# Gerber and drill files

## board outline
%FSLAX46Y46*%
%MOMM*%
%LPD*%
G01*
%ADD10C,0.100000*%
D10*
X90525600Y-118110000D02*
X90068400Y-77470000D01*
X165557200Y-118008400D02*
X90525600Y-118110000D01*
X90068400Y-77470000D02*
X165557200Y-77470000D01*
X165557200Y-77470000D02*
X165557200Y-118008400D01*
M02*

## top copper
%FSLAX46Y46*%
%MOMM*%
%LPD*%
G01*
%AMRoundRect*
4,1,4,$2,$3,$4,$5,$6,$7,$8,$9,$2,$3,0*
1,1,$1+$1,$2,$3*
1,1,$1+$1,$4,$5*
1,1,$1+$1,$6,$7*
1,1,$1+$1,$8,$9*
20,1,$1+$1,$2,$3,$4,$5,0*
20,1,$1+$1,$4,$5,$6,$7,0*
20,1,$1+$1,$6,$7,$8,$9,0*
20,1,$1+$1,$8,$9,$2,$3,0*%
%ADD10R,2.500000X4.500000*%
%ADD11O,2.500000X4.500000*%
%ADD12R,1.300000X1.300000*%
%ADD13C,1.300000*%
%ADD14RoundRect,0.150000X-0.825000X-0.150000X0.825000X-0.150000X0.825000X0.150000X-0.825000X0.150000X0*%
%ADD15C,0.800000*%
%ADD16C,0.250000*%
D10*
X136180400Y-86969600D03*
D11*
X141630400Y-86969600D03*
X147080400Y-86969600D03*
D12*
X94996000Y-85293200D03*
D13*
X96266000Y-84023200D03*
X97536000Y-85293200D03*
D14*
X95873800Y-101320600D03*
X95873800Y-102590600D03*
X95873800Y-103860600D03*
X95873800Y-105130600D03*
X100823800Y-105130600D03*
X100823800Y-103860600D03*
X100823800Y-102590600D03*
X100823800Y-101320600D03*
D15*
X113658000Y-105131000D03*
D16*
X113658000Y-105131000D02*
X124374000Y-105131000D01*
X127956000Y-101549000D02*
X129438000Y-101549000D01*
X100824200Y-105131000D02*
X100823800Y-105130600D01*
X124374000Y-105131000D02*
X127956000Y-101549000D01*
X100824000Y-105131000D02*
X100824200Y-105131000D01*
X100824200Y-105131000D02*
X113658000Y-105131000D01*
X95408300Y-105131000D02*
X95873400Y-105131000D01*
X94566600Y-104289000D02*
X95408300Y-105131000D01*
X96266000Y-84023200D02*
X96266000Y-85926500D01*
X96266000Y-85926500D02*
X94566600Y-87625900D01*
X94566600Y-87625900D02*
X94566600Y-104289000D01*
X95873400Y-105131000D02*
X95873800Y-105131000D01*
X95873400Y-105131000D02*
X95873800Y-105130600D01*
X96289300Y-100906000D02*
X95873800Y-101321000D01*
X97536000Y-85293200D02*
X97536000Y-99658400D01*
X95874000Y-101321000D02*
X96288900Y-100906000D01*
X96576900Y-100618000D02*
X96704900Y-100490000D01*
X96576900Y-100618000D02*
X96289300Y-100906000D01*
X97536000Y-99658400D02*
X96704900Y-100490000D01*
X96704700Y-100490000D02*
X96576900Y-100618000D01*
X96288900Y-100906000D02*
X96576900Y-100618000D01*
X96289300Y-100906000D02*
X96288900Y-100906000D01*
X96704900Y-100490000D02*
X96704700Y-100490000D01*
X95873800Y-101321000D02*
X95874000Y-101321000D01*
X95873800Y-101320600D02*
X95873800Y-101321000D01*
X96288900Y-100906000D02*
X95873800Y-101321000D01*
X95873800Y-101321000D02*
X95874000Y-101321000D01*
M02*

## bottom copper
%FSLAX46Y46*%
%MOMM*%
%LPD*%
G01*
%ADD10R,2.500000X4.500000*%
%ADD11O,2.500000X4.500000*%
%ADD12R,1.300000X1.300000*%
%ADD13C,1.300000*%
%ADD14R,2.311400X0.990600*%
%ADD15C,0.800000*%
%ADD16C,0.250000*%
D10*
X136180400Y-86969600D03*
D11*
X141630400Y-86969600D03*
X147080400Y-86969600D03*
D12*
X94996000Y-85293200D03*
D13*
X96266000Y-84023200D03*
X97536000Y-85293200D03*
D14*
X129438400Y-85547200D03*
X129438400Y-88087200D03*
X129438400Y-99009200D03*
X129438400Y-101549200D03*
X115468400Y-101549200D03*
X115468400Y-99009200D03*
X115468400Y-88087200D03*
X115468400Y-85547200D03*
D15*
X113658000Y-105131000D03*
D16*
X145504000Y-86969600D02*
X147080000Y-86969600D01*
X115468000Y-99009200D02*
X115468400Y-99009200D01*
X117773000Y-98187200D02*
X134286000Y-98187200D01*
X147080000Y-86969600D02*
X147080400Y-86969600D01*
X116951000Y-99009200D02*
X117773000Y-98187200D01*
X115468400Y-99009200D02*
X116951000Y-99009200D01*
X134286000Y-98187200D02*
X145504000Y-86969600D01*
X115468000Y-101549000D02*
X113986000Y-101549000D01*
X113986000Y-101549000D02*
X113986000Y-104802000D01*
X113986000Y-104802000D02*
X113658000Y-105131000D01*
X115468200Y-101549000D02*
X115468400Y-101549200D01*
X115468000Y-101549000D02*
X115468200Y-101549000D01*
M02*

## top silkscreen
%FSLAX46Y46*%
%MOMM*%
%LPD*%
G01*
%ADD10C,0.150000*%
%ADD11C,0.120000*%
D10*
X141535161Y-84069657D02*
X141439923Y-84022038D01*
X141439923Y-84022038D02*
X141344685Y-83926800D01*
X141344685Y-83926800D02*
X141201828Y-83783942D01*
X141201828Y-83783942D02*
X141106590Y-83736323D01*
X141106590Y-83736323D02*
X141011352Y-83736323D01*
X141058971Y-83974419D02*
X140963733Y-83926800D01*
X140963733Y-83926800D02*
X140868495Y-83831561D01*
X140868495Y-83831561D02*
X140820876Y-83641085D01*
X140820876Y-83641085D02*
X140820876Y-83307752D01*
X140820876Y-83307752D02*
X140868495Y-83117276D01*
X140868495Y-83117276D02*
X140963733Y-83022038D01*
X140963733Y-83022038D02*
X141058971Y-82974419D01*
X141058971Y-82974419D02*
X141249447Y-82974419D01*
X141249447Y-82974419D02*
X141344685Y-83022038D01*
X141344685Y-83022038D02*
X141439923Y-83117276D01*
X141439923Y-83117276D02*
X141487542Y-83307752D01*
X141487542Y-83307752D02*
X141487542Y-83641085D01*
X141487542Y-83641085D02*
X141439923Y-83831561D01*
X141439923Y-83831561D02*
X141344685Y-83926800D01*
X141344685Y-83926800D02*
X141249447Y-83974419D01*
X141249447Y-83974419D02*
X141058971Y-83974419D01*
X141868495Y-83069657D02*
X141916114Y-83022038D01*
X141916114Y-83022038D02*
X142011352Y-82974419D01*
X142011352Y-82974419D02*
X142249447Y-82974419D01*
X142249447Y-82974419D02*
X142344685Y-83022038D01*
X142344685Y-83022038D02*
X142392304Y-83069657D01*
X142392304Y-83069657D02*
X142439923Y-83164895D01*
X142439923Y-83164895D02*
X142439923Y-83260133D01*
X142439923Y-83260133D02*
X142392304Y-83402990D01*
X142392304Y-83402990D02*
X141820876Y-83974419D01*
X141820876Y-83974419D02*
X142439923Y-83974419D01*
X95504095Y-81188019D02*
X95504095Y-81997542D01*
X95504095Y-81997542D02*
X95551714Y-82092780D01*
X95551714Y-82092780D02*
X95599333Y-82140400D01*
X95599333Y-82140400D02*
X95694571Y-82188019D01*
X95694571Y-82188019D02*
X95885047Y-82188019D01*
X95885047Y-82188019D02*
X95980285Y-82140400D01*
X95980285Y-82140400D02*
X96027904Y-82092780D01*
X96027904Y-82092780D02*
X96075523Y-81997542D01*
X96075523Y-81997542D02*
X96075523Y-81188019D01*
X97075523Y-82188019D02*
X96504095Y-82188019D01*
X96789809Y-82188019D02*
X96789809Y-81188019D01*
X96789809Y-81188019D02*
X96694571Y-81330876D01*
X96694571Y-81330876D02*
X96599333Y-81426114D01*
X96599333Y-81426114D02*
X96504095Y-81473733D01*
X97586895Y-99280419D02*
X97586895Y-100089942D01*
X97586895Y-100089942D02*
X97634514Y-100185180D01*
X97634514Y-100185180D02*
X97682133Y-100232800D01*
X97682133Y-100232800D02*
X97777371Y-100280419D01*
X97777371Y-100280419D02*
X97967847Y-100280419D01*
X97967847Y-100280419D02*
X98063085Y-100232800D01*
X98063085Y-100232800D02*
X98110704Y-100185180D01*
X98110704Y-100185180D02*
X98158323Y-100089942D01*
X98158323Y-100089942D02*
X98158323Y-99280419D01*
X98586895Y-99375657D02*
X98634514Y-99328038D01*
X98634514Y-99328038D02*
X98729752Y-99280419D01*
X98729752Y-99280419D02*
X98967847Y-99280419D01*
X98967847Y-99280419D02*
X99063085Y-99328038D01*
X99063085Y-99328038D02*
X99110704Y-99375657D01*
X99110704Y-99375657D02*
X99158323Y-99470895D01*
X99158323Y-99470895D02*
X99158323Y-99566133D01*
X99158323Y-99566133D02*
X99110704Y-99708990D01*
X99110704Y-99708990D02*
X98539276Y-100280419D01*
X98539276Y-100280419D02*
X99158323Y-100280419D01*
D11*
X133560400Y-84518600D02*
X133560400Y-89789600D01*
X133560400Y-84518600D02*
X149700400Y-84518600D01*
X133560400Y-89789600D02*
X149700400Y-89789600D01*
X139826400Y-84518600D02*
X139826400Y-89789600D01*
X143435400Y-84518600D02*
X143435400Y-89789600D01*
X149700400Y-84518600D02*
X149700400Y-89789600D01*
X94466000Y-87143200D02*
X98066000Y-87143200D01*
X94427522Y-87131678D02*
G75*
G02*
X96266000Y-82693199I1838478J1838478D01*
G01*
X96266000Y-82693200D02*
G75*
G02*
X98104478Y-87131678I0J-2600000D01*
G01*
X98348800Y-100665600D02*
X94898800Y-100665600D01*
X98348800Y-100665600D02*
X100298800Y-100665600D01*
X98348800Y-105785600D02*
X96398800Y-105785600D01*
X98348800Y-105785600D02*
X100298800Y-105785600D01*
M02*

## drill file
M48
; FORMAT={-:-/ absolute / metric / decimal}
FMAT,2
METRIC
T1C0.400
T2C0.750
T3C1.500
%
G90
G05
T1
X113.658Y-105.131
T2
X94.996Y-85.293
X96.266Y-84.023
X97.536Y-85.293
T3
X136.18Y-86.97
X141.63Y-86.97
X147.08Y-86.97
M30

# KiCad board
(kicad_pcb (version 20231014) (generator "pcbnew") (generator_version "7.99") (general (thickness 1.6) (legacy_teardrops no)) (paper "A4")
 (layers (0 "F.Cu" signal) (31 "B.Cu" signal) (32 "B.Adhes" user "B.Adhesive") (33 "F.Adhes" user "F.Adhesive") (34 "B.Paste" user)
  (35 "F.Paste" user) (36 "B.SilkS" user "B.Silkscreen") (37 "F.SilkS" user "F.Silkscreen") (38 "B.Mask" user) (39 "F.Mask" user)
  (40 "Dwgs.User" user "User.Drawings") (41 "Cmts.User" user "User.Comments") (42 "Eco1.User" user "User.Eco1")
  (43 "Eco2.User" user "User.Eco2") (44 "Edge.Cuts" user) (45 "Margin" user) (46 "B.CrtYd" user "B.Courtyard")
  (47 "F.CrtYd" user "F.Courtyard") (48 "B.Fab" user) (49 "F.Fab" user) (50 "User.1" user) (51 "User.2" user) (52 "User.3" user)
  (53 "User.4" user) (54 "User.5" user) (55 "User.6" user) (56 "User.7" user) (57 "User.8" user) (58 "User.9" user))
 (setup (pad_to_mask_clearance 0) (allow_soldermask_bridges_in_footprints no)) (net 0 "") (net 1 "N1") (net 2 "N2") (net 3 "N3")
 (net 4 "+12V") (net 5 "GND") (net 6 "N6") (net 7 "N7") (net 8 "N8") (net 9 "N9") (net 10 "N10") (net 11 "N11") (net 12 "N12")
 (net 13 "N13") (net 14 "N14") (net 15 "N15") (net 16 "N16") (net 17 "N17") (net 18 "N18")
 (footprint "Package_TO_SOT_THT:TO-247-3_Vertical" (layer "F.Cu") (at 136.1804 86.9696)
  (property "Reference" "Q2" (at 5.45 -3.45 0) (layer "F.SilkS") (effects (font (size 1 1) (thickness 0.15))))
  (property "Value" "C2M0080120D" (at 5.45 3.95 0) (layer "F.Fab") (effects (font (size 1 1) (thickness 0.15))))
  (fp_line (start -2.62 -2.451) (end -2.62 2.82) (stroke (width 0.12) (type solid)) (layer "F.SilkS"))
  (fp_line (start -2.62 -2.451) (end 13.52 -2.451) (stroke (width 0.12) (type solid)) (layer "F.SilkS"))
  (fp_line (start -2.62 2.82) (end 13.52 2.82) (stroke (width 0.12) (type solid)) (layer "F.SilkS"))
  (fp_line (start 3.646 -2.451) (end 3.646 2.82) (stroke (width 0.12) (type solid)) (layer "F.SilkS"))
  (fp_line (start 7.255 -2.451) (end 7.255 2.82) (stroke (width 0.12) (type solid)) (layer "F.SilkS"))
  (fp_line (start 13.52 -2.451) (end 13.52 2.82) (stroke (width 0.12) (type solid)) (layer "F.SilkS"))
  (pad "1" thru_hole rect (at 0 0) (size 2.5 4.5) (drill 1.5) (layers "*.Cu" "*.Mask") (remove_unused_layers no) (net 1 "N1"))
  (pad "2" thru_hole oval (at 5.45 0) (size 2.5 4.5) (drill 1.5) (layers "*.Cu" "*.Mask") (remove_unused_layers no) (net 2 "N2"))
  (pad "3" thru_hole oval (at 10.9 0) (size 2.5 4.5) (drill 1.5) (layers "*.Cu" "*.Mask") (remove_unused_layers no) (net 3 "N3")))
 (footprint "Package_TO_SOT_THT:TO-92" (layer "F.Cu") (at 94.996 85.2932)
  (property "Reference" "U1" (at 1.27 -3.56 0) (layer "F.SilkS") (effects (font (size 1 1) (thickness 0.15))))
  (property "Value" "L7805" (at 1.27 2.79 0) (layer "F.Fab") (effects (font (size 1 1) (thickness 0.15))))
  (fp_line (start -0.53 1.85) (end 3.07 1.85) (stroke (width 0.12) (type solid)) (layer "F.SilkS"))
  (fp_arc (start -0.568478 1.838478) (mid -1.132087 -0.994977) (end 1.27 -2.6) (stroke (width 0.12) (type solid)) (layer "F.SilkS"))
  (fp_arc (start 1.27 -2.6) (mid 3.672087 -0.994977) (end 3.108478 1.838478) (stroke (width 0.12) (type solid)) (layer "F.SilkS"))
  (pad "1" thru_hole rect (at 0 0) (size 1.3 1.3) (drill 0.75) (layers "*.Cu" "*.Mask") (remove_unused_layers no) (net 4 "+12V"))
  (pad "2" thru_hole circle (at 1.27 -1.27) (size 1.3 1.3) (drill 0.75) (layers "*.Cu" "*.Mask") (remove_unused_layers no) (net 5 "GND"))
  (pad "3" thru_hole circle (at 2.54 0) (size 1.3 1.3) (drill 0.75) (layers "*.Cu" "*.Mask") (remove_unused_layers no) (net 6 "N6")))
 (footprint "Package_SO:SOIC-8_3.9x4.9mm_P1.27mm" (layer "F.Cu") (at 98.3488 103.2256)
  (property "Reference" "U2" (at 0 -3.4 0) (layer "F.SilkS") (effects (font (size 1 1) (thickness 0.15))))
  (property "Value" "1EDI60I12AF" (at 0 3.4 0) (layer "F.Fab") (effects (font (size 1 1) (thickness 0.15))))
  (fp_line (start 0 -2.56) (end -3.45 -2.56) (stroke (width 0.12) (type solid)) (layer "F.SilkS"))
  (fp_line (start 0 -2.56) (end 1.95 -2.56) (stroke (width 0.12) (type solid)) (layer "F.SilkS"))
  (fp_line (start 0 2.56) (end -1.95 2.56) (stroke (width 0.12) (type solid)) (layer "F.SilkS"))
  (fp_line (start 0 2.56) (end 1.95 2.56) (stroke (width 0.12) (type solid)) (layer "F.SilkS"))
  (pad "1" smd roundrect (at -2.475 -1.905) (size 1.95 0.6) (layers "F.Cu" "F.Paste" "F.Mask") (roundrect_rratio 0.25) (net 6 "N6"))
  (pad "2" smd roundrect (at -2.475 -0.635) (size 1.95 0.6) (layers "F.Cu" "F.Paste" "F.Mask") (roundrect_rratio 0.25) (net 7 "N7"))
  (pad "3" smd roundrect (at -2.475 0.635) (size 1.95 0.6) (layers "F.Cu" "F.Paste" "F.Mask") (roundrect_rratio 0.25) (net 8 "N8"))
  (pad "4" smd roundrect (at -2.475 1.905) (size 1.95 0.6) (layers "F.Cu" "F.Paste" "F.Mask") (roundrect_rratio 0.25) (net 5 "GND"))
  (pad "5" smd roundrect (at 2.475 1.905) (size 1.95 0.6) (layers "F.Cu" "F.Paste" "F.Mask") (roundrect_rratio 0.25) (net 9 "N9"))
  (pad "6" smd roundrect (at 2.475 0.635) (size 1.95 0.6) (layers "F.Cu" "F.Paste" "F.Mask") (roundrect_rratio 0.25) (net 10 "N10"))
  (pad "7" smd roundrect (at 2.475 -0.635) (size 1.95 0.6) (layers "F.Cu" "F.Paste" "F.Mask") (roundrect_rratio 0.25) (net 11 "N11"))
  (pad "8" smd roundrect (at 2.475 -1.905) (size 1.95 0.6) (layers "F.Cu" "F.Paste" "F.Mask") (roundrect_rratio 0.25) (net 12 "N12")))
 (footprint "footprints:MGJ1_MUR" (layer "B.Cu") (at 122.4534 94.4367 180)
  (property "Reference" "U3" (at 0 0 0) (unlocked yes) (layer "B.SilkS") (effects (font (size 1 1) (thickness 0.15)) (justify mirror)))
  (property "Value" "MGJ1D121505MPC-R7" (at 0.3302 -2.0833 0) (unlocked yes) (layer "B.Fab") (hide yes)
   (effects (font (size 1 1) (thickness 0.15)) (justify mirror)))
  (pad "1" smd rect (at -6.985 8.8895 180) (size 2.3114 0.9906) (layers "B.Cu" "B.Paste" "B.Mask") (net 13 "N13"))
  (pad "2" smd rect (at -6.985 6.3495 180) (size 2.3114 0.9906) (layers "B.Cu" "B.Paste" "B.Mask") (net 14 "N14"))
  (pad "3" smd rect (at -6.985 -4.5725 180) (size 2.3114 0.9906) (layers "B.Cu" "B.Paste" "B.Mask") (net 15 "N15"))
  (pad "4" smd rect (at -6.985 -7.1125 180) (size 2.3114 0.9906) (layers "B.Cu" "B.Paste" "B.Mask") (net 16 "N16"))
  (pad "5" smd rect (at 6.985 -7.1125 180) (size 2.3114 0.9906) (layers "B.Cu" "B.Paste" "B.Mask") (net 9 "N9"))
  (pad "6" smd rect (at 6.985 -4.5725 180) (size 2.3114 0.9906) (layers "B.Cu" "B.Paste" "B.Mask") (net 3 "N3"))
  (pad "7" smd rect (at 6.985 6.3495 180) (size 2.3114 0.9906) (layers "B.Cu" "B.Paste" "B.Mask") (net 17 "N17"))
  (pad "8" smd rect (at 6.985 8.8895 180) (size 2.3114 0.9906) (layers "B.Cu" "B.Paste" "B.Mask") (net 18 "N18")))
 (gr_line (start 90.5256 118.11) (end 90.0684 77.47) (stroke (width 0.1) (type default)) (layer "Edge.Cuts"))
 (gr_line (start 165.5572 118.0084) (end 90.5256 118.11) (stroke (width 0.1) (type default)) (layer "Edge.Cuts"))
 (gr_line (start 90.0684 77.47) (end 165.5572 77.47) (stroke (width 0.1) (type default)) (layer "Edge.Cuts"))
 (gr_line (start 165.5572 77.47) (end 165.5572 118.0084) (stroke (width 0.1) (type default)) (layer "Edge.Cuts"))
 (segment (start 145.504 86.9696) (end 147.08 86.9696) (width 0.25) (layer "B.Cu") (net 3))
 (segment (start 115.468 99.0092) (end 115.4684 99.0092) (width 0.25) (layer "B.Cu") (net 3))
 (segment (start 117.773 98.1872) (end 134.286 98.1872) (width 0.25) (layer "B.Cu") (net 3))
 (segment (start 147.08 86.9696) (end 147.0804 86.9696) (width 0.25) (layer "B.Cu") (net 3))
 (segment (start 116.951 99.0092) (end 117.773 98.1872) (width 0.25) (layer "B.Cu") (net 3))
 (segment (start 115.4684 99.0092) (end 116.951 99.0092) (width 0.25) (layer "B.Cu") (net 3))
 (segment (start 134.286 98.1872) (end 145.504 86.9696) (width 0.25) (layer "B.Cu") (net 3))
 (segment (start 113.658 105.131) (end 124.374 105.131) (width 0.25) (layer "F.Cu") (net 9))
 (segment (start 127.956 101.549) (end 129.438 101.549) (width 0.25) (layer "F.Cu") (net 9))
 (segment (start 100.8242 105.131) (end 100.8238 105.1306) (width 0.25) (layer "F.Cu") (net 9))
 (segment (start 124.374 105.131) (end 127.956 101.549) (width 0.25) (layer "F.Cu") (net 9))
 (segment (start 100.824 105.131) (end 100.8242 105.131) (width 0.25) (layer "F.Cu") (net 9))
 (segment (start 100.8242 105.131) (end 113.658 105.131) (width 0.25) (layer "F.Cu") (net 9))
 (via (at 113.658 105.131) (size 0.8) (drill 0.4) (layers "F.Cu" "B.Cu") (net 9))
 (segment (start 115.468 101.549) (end 113.986 101.549) (width 0.25) (layer "B.Cu") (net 9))
 (segment (start 113.986 101.549) (end 113.986 104.802) (width 0.25) (layer "B.Cu") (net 9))
 (segment (start 113.986 104.802) (end 113.658 105.131) (width 0.25) (layer "B.Cu") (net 9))
 (segment (start 115.4682 101.549) (end 115.4684 101.5492) (width 0.25) (layer "B.Cu") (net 9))
 (segment (start 115.468 101.549) (end 115.4682 101.549) (width 0.25) (layer "B.Cu") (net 9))
 (segment (start 95.4083 105.131) (end 95.8734 105.131) (width 0.25) (layer "F.Cu") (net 5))
 (segment (start 94.5666 104.289) (end 95.4083 105.131) (width 0.25) (layer "F.Cu") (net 5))
 (segment (start 96.266 84.0232) (end 96.266 85.9265) (width 0.25) (layer "F.Cu") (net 5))
 (segment (start 96.266 85.9265) (end 94.5666 87.6259) (width 0.25) (layer "F.Cu") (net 5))
 (segment (start 94.5666 87.6259) (end 94.5666 104.289) (width 0.25) (layer "F.Cu") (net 5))
 (segment (start 95.8734 105.131) (end 95.8738 105.131) (width 0.25) (layer "F.Cu") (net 5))
 (segment (start 95.8734 105.131) (end 95.8738 105.1306) (width 0.25) (layer "F.Cu") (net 5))
 (segment (start 96.2893 100.906) (end 95.8738 101.321) (width 0.25) (layer "F.Cu") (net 6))
 (segment (start 97.536 85.2932) (end 97.536 99.6584) (width 0.25) (layer "F.Cu") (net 6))
 (segment (start 95.874 101.321) (end 96.2889 100.906) (width 0.25) (layer "F.Cu") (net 6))
 (segment (start 96.5769 100.618) (end 96.7049 100.49) (width 0.25) (layer "F.Cu") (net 6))
 (segment (start 96.5769 100.618) (end 96.2893 100.906) (width 0.25) (layer "F.Cu") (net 6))
 (segment (start 97.536 99.6584) (end 96.7049 100.49) (width 0.25) (layer "F.Cu") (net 6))
 (segment (start 96.7047 100.49) (end 96.5769 100.618) (width 0.25) (layer "F.Cu") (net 6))
 (segment (start 96.2889 100.906) (end 96.5769 100.618) (width 0.25) (layer "F.Cu") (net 6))
 (segment (start 96.2893 100.906) (end 96.2889 100.906) (width 0.25) (layer "F.Cu") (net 6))
 (segment (start 96.7049 100.49) (end 96.7047 100.49) (width 0.25) (layer "F.Cu") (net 6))
 (segment (start 95.8738 101.321) (end 95.874 101.321) (width 0.25) (layer "F.Cu") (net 6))
 (segment (start 95.8738 101.3206) (end 95.8738 101.321) (width 0.25) (layer "F.Cu") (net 6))
 (segment (start 96.2889 100.906) (end 95.8738 101.321) (width 0.25) (layer "F.Cu") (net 6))
 (segment (start 95.8738 101.321) (end 95.874 101.321) (width 0.25) (layer "F.Cu") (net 6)))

